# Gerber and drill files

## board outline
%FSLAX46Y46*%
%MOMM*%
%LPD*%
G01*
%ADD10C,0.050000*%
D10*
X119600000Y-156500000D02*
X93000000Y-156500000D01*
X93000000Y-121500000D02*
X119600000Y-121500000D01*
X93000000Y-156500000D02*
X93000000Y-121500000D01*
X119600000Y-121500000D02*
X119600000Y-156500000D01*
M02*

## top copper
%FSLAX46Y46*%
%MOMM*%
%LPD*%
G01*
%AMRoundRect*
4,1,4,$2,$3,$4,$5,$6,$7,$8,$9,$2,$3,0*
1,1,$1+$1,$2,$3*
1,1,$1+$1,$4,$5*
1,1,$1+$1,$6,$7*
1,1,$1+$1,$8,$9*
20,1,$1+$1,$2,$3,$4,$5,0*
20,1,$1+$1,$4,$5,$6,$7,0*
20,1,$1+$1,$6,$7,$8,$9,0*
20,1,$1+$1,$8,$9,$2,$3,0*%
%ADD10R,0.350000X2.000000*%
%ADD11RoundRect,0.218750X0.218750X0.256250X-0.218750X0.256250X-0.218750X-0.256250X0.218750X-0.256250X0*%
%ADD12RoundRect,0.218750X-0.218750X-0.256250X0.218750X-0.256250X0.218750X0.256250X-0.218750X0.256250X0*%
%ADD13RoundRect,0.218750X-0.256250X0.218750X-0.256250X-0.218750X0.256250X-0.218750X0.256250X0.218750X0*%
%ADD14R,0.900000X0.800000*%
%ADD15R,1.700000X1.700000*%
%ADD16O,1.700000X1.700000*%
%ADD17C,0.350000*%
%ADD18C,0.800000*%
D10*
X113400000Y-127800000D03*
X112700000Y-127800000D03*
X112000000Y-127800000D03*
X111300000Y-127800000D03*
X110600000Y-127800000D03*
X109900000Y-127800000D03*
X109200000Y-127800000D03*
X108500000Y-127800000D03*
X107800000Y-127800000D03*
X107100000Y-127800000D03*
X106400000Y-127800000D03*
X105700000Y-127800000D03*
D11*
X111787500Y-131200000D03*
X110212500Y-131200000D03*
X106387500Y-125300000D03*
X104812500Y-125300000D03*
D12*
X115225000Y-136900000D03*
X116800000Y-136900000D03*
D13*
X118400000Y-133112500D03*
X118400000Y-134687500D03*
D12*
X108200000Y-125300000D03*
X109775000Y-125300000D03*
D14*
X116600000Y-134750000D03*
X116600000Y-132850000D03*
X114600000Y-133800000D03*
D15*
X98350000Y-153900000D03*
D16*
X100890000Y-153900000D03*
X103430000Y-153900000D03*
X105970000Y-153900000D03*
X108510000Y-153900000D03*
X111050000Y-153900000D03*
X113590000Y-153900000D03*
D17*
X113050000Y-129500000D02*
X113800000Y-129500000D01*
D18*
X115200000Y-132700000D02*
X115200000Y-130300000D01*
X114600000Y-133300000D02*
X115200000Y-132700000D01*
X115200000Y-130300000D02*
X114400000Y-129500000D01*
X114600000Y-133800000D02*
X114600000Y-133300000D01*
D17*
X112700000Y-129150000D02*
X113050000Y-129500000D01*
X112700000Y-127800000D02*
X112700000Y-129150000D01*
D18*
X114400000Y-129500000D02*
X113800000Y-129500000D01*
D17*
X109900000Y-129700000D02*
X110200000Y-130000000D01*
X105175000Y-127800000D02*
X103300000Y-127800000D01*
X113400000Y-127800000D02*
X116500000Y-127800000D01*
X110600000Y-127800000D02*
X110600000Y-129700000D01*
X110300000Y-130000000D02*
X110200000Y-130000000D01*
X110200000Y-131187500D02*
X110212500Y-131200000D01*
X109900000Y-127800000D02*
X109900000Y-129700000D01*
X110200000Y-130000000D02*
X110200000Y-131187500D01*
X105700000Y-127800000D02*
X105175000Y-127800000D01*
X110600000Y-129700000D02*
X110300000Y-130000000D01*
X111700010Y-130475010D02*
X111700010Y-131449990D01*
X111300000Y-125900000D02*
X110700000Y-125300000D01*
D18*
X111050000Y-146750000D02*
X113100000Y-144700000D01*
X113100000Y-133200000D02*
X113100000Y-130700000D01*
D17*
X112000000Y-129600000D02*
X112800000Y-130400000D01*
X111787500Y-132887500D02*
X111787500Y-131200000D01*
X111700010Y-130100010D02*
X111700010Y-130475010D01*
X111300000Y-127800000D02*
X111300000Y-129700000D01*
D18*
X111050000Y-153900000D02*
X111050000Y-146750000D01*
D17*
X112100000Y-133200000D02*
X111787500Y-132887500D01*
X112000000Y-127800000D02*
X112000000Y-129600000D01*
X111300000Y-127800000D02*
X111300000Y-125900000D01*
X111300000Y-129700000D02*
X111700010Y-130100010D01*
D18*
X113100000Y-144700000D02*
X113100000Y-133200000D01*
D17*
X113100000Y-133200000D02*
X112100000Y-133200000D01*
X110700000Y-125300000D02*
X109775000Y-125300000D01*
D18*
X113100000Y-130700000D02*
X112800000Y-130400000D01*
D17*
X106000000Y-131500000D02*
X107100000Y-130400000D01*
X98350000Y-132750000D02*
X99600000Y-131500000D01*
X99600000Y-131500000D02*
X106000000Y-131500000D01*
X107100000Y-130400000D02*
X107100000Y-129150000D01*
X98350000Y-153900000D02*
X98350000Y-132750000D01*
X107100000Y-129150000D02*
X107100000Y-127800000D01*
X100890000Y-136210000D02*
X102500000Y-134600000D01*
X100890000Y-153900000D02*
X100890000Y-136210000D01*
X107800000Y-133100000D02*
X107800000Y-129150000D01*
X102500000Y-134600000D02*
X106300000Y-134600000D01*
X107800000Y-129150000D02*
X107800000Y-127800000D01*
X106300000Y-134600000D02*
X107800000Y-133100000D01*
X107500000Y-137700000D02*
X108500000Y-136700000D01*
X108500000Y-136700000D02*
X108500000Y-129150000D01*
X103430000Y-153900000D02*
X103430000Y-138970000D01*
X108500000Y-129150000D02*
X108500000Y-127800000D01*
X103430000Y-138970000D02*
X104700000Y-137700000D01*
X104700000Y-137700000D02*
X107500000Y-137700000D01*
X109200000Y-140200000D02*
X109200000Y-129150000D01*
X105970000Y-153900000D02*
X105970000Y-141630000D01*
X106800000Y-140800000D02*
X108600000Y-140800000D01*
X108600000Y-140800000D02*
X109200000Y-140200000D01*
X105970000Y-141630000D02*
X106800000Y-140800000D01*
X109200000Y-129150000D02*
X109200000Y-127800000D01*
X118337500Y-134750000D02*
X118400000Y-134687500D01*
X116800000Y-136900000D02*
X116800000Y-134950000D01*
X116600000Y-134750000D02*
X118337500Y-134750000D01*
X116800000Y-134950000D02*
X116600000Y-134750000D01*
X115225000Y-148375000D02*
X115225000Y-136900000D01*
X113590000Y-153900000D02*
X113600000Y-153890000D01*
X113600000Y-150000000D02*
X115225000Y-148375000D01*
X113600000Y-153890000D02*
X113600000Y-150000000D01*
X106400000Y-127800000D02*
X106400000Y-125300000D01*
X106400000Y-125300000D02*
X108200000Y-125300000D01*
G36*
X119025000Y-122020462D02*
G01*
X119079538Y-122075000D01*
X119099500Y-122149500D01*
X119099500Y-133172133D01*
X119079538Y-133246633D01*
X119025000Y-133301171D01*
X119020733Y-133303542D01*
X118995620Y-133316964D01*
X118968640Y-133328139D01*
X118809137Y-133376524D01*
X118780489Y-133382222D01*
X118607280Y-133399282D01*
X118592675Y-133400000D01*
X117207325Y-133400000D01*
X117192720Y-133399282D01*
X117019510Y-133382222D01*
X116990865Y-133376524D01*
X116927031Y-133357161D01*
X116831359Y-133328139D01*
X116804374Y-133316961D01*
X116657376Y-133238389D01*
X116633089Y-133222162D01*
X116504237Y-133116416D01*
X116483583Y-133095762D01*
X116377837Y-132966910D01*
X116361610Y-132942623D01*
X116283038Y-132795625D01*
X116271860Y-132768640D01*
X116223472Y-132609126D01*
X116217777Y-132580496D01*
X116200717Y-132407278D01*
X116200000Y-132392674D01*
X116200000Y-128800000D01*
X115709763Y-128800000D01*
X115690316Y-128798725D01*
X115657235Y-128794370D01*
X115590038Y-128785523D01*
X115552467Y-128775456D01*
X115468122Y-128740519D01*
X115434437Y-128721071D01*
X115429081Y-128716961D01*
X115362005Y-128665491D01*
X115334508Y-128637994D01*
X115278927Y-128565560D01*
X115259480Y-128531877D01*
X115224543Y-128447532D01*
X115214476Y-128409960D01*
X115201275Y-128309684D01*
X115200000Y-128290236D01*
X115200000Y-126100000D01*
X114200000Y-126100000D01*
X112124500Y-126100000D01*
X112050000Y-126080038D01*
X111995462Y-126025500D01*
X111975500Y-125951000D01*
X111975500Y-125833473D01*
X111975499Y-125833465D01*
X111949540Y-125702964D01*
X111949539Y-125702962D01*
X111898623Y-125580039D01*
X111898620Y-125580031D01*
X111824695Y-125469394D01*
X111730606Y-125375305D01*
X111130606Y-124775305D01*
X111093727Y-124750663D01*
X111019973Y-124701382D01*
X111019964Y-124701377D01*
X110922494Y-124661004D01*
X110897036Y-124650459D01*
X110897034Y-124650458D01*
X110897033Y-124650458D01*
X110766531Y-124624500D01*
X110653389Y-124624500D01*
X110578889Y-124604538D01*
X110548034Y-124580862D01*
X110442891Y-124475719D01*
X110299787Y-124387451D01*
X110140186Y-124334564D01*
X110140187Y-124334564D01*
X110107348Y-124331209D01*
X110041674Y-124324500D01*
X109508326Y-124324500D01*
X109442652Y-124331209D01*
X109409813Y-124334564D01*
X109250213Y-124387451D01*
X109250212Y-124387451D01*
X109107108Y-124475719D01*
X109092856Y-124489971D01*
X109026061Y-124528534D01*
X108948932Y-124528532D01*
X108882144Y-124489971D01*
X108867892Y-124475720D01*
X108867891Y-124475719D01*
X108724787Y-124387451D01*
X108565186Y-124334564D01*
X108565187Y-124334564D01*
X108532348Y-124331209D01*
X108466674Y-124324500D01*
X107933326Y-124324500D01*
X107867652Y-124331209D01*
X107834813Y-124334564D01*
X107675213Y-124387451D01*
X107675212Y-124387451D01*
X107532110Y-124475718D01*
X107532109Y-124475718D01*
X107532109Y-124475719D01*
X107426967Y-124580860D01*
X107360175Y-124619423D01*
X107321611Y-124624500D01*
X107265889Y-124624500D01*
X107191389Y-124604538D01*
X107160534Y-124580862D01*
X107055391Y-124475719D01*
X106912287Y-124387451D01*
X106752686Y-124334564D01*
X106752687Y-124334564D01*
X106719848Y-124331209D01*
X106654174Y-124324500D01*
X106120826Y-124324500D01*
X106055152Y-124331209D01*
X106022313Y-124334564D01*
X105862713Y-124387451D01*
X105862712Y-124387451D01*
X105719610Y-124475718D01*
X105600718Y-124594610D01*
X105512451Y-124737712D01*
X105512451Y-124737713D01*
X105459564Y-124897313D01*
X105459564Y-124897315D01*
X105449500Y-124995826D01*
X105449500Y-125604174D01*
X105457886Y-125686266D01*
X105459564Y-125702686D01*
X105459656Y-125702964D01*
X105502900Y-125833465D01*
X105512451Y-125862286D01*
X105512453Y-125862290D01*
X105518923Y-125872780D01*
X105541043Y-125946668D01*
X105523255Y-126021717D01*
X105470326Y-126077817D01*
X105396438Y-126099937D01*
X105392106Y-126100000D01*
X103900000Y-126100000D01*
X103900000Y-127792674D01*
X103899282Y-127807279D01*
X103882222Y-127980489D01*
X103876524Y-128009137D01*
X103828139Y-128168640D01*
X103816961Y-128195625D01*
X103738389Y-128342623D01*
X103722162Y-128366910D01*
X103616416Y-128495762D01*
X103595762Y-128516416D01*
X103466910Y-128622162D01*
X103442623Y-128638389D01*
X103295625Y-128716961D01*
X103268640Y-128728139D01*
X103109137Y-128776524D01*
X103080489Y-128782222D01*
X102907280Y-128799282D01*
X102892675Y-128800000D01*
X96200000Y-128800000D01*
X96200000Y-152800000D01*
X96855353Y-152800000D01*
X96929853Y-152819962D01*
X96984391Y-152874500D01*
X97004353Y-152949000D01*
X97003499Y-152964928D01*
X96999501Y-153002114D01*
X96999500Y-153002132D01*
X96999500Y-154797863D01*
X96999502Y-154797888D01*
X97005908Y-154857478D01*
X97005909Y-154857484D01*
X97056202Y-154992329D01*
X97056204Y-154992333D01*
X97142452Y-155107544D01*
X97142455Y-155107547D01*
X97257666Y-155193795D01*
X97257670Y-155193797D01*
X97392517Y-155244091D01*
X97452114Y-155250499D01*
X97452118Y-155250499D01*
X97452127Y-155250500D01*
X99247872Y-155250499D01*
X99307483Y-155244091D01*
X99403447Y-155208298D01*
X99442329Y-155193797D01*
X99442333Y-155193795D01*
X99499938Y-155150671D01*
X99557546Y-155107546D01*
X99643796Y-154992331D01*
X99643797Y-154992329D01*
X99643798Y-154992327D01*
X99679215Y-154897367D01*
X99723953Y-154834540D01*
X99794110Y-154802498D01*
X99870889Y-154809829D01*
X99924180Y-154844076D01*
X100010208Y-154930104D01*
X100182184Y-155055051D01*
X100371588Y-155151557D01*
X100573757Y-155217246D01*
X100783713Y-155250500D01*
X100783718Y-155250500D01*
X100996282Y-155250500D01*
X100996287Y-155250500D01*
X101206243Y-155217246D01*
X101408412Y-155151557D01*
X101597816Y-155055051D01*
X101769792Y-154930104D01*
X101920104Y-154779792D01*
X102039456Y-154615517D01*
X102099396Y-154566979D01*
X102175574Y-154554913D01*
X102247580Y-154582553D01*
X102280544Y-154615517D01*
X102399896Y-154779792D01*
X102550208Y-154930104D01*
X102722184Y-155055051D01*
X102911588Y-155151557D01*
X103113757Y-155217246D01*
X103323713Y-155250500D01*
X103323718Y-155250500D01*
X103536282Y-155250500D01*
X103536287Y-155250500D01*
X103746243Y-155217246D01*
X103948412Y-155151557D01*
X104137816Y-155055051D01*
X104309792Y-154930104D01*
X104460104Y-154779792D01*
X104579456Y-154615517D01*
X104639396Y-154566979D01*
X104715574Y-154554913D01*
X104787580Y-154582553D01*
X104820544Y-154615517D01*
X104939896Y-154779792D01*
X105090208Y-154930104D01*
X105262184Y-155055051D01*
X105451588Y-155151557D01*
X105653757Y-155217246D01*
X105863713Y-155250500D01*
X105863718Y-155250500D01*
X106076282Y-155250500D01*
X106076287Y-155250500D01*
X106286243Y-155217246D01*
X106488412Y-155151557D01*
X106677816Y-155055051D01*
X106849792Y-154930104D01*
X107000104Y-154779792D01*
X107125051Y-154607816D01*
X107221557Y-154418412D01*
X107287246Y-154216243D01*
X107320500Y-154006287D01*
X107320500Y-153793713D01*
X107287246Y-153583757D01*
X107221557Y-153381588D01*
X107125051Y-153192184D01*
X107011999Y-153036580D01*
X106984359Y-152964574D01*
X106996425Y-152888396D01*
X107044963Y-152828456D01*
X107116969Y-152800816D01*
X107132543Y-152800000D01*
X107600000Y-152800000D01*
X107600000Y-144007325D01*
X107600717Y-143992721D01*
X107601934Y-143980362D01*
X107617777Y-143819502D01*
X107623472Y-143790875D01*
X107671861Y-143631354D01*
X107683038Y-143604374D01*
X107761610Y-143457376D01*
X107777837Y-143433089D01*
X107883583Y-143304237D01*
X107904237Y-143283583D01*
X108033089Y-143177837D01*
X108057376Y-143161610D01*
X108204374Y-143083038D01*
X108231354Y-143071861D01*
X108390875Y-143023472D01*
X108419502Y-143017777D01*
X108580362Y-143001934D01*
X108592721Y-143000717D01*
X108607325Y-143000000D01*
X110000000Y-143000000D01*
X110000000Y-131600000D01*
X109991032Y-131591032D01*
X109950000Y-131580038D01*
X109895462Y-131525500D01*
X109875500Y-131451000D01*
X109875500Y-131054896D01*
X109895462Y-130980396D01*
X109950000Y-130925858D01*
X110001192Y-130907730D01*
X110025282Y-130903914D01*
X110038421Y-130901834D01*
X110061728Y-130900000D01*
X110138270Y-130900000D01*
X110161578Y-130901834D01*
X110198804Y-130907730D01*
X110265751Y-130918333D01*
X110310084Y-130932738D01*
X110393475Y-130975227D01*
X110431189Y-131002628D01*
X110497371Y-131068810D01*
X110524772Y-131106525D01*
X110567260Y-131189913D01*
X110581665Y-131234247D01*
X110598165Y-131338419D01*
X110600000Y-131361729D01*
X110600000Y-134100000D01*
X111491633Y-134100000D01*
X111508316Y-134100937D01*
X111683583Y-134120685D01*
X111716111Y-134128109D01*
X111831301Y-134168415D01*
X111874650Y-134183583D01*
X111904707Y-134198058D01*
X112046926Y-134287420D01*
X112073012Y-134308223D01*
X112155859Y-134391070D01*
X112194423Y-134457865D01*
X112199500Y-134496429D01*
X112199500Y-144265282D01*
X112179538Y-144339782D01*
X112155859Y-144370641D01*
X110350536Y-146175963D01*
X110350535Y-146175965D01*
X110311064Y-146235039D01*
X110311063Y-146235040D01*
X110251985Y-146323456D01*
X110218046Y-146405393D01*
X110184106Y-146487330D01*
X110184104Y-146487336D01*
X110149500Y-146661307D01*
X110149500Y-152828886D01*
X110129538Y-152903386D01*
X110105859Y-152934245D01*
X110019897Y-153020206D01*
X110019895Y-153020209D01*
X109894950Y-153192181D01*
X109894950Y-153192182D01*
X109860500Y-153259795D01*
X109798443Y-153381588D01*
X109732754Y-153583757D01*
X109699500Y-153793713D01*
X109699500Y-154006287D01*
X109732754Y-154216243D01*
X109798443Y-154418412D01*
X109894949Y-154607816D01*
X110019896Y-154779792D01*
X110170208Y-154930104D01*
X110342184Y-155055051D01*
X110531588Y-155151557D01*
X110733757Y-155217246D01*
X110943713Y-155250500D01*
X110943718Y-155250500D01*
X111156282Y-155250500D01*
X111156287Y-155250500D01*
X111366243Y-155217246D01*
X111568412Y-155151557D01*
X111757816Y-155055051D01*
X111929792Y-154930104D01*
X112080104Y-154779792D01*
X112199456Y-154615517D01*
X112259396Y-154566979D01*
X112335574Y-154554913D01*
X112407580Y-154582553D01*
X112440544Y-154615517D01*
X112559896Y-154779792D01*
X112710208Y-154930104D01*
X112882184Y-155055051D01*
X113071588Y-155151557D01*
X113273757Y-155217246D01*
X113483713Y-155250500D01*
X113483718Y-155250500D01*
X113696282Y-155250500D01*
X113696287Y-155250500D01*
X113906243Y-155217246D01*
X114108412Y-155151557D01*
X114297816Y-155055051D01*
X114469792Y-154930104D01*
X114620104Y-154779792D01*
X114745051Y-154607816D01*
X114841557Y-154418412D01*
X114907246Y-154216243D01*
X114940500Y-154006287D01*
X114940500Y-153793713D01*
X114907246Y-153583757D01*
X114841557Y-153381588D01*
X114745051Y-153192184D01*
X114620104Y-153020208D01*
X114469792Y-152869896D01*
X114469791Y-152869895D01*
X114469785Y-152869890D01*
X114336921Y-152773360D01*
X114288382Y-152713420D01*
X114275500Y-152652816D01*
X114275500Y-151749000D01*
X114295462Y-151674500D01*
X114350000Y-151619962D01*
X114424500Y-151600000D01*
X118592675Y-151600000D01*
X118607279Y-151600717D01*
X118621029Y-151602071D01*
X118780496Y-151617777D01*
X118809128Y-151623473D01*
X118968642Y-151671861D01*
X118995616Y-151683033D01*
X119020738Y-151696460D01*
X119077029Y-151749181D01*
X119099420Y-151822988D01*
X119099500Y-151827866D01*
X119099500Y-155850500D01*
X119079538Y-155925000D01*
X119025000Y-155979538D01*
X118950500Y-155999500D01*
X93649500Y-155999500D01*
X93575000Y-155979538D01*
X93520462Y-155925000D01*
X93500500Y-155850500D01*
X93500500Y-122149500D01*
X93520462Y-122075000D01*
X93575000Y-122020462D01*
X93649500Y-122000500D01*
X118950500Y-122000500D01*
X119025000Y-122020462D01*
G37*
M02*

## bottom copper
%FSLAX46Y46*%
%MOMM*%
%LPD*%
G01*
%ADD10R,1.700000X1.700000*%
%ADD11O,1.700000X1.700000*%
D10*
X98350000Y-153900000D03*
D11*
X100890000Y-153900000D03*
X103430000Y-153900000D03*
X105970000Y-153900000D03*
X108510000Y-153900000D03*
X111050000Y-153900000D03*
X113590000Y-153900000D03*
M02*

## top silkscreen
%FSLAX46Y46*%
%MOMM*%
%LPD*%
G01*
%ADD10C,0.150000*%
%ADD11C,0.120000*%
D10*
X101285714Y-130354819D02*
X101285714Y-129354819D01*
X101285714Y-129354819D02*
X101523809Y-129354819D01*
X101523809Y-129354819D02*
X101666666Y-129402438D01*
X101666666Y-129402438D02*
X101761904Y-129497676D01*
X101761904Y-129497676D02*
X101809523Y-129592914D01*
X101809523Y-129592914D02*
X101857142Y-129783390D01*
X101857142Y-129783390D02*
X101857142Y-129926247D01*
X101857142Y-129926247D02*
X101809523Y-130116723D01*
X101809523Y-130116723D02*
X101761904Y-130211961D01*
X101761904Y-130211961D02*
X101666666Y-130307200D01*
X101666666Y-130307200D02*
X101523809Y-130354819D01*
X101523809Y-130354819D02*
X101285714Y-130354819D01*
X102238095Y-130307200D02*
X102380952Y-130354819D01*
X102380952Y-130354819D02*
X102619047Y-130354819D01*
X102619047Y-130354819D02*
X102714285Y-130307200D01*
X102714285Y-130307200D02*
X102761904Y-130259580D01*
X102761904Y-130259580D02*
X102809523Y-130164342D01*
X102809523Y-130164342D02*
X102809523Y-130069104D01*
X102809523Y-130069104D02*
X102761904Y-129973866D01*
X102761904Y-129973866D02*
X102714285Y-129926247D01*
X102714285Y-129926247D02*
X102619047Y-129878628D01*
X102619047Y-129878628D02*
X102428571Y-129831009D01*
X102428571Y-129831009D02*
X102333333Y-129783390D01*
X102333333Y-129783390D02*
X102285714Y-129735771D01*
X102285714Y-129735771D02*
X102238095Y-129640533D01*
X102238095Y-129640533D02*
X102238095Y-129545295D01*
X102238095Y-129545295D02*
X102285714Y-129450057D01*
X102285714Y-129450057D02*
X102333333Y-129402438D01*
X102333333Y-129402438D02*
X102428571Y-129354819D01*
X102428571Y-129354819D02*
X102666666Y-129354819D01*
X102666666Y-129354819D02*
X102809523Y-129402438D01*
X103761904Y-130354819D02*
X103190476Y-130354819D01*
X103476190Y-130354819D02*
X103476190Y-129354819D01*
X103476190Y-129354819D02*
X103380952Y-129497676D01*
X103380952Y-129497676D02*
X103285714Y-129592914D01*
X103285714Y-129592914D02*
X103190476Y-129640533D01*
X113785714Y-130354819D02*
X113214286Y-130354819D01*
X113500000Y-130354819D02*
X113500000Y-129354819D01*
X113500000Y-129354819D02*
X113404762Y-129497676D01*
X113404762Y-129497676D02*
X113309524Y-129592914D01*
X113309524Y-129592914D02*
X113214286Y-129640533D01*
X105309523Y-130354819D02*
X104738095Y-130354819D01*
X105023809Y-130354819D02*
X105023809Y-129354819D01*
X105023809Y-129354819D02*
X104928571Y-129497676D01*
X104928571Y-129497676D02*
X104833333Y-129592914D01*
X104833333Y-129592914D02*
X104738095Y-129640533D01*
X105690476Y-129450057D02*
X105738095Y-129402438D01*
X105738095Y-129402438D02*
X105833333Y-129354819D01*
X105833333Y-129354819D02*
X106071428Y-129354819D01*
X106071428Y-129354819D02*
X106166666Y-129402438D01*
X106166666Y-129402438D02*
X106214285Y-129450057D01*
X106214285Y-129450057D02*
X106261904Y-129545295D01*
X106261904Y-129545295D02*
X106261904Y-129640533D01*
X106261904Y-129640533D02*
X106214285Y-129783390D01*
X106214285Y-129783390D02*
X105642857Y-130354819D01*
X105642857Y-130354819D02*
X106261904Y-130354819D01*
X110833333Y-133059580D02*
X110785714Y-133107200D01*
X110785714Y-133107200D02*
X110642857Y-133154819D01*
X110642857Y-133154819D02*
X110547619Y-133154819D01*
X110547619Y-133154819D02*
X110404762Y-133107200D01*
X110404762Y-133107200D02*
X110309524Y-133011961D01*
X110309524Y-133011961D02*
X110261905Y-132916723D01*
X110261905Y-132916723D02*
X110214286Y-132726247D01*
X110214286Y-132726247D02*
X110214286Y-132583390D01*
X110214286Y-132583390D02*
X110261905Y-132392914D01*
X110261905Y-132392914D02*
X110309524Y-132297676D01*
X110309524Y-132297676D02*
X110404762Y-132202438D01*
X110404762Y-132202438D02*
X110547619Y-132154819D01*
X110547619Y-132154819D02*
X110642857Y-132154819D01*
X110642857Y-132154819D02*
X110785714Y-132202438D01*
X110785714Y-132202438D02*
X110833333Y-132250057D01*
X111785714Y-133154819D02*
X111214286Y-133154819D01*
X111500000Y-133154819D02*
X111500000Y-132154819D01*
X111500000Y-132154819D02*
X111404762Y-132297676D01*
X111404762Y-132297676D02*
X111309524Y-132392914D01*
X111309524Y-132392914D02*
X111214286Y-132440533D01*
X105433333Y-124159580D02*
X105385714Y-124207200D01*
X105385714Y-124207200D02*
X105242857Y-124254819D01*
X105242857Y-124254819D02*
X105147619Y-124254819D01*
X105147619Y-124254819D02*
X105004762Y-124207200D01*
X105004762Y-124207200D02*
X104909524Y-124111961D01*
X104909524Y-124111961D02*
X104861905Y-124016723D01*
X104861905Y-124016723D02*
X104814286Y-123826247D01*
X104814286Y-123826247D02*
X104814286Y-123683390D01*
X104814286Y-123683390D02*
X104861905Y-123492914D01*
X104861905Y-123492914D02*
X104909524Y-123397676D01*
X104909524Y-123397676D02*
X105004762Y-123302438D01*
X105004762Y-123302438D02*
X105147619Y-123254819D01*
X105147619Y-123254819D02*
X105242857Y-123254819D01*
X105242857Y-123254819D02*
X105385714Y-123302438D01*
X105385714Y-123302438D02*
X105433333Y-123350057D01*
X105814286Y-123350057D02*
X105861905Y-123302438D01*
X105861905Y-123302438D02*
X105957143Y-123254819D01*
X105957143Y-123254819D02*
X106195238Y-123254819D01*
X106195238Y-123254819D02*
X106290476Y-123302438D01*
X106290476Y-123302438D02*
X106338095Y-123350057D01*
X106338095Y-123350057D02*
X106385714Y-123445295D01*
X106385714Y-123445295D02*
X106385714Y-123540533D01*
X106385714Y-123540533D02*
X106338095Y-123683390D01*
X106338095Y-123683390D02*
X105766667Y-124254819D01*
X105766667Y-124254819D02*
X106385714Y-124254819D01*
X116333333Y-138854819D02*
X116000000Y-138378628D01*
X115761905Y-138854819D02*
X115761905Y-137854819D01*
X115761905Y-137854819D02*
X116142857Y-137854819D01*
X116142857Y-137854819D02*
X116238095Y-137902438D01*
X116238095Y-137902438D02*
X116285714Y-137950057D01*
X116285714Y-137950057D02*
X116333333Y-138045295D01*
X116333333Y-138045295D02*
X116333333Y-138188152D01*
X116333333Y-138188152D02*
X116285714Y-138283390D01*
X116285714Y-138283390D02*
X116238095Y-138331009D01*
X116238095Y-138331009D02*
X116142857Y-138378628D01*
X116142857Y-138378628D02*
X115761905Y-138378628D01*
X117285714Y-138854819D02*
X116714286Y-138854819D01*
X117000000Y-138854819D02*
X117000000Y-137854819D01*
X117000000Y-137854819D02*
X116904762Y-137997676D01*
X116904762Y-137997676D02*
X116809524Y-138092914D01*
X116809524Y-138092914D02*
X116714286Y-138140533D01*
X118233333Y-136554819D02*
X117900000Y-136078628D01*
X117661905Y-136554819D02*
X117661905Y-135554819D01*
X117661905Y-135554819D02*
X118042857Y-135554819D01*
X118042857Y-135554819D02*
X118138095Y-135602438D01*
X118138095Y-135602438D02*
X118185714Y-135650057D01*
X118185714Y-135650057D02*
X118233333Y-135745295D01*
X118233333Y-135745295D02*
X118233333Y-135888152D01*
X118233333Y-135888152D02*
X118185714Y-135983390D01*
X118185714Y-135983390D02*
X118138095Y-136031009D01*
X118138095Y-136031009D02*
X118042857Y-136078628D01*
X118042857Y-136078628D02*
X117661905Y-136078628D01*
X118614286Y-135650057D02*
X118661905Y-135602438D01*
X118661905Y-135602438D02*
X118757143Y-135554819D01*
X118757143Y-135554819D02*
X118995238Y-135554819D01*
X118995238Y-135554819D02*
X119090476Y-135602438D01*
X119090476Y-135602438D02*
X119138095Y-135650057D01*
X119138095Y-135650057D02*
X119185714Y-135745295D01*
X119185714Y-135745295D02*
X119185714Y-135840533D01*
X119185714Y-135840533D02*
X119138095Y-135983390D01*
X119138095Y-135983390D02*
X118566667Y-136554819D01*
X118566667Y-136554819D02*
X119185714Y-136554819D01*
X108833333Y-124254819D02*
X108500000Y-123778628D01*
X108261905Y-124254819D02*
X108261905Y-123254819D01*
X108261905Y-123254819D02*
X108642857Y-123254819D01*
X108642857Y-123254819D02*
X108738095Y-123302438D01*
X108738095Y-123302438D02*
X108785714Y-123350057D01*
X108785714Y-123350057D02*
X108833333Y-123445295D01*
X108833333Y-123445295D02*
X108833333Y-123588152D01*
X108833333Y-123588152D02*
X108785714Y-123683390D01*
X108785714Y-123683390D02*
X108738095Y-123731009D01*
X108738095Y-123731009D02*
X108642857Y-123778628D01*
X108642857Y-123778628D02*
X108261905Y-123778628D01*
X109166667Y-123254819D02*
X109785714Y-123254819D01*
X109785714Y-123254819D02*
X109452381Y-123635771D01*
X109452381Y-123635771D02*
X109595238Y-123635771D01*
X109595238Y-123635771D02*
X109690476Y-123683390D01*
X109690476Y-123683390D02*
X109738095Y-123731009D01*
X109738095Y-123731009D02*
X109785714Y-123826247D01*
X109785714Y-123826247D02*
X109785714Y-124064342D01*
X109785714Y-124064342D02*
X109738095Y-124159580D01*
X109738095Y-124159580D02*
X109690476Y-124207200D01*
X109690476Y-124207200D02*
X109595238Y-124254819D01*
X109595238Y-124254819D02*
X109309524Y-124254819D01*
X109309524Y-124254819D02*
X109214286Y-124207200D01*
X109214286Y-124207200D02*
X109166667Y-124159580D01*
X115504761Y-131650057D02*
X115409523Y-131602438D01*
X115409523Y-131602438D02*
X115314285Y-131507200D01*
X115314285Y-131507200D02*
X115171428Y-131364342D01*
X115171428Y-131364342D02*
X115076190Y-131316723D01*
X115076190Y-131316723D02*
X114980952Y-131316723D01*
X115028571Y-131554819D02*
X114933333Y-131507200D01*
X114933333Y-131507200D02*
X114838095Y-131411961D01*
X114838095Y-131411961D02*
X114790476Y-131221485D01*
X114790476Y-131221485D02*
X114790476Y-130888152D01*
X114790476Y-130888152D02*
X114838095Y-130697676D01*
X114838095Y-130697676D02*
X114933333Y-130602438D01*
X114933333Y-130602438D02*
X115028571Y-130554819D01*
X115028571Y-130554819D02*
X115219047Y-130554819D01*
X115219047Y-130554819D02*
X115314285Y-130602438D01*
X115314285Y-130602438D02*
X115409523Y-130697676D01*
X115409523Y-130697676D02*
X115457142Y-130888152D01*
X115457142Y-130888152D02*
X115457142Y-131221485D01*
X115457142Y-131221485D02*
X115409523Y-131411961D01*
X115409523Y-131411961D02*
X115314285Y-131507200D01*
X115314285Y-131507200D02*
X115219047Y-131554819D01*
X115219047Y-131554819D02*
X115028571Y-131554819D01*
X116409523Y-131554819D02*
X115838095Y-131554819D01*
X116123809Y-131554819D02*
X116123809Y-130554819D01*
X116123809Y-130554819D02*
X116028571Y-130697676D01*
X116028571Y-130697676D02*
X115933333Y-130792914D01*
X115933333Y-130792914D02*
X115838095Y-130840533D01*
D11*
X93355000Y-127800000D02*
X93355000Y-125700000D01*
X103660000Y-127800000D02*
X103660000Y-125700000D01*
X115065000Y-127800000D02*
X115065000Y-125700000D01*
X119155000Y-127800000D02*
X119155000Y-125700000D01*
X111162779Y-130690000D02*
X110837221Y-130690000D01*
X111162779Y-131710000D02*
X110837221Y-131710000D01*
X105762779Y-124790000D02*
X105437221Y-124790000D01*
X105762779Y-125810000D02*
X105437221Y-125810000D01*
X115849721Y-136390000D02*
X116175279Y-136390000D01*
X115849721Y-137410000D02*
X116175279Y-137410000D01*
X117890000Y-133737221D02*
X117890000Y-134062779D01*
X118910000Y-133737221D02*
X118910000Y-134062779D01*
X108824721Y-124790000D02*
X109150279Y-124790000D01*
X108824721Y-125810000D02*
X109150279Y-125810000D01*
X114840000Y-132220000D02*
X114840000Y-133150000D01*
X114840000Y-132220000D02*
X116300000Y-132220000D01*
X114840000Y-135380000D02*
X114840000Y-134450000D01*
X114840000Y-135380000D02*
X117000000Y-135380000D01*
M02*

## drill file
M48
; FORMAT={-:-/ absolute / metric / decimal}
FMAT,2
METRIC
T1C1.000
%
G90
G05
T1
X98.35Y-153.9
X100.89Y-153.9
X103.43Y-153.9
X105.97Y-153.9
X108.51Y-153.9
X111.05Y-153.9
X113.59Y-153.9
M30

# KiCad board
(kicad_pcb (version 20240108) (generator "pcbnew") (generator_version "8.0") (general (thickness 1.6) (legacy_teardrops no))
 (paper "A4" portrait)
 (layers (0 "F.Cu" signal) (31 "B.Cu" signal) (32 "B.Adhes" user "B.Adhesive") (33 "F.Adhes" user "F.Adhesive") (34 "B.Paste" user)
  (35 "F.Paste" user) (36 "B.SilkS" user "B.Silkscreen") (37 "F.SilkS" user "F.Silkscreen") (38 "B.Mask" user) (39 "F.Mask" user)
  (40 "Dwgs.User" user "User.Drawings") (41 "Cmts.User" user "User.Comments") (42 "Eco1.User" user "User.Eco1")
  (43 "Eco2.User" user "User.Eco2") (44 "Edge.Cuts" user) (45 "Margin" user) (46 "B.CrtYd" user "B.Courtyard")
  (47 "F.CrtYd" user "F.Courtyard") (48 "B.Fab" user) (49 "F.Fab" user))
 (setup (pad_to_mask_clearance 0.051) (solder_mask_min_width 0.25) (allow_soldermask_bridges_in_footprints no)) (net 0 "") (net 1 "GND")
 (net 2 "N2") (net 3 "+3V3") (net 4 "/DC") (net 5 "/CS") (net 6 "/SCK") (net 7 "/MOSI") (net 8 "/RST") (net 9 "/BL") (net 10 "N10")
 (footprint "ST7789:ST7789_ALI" (layer "F.Cu") (at 109.9 124.3)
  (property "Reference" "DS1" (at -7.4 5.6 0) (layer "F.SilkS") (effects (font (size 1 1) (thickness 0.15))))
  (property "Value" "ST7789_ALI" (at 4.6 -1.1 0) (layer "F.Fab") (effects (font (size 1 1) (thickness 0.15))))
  (fp_line (start -16.545 3.5) (end -16.545 1.4) (stroke (width 0.12) (type solid)) (layer "F.SilkS"))
  (fp_line (start -6.24 3.5) (end -6.24 1.4) (stroke (width 0.12) (type solid)) (layer "F.SilkS"))
  (fp_line (start 5.165 3.5) (end 5.165 1.4) (stroke (width 0.12) (type solid)) (layer "F.SilkS"))
  (fp_line (start 9.255 3.5) (end 9.255 1.4) (stroke (width 0.12) (type solid)) (layer "F.SilkS"))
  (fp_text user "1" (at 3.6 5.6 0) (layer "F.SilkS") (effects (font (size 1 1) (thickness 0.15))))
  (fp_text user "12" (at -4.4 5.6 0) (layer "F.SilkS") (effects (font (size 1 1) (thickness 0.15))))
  (pad "1" smd rect (at 3.5 3.5) (size 0.35 2) (layers "F.Cu" "F.Paste" "F.Mask") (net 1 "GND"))
  (pad "2" smd rect (at 2.8 3.5) (size 0.35 2) (layers "F.Cu" "F.Paste" "F.Mask") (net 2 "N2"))
  (pad "3" smd rect (at 2.1 3.5) (size 0.35 2) (layers "F.Cu" "F.Paste" "F.Mask") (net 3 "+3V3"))
  (pad "4" smd rect (at 1.4 3.5) (size 0.35 2) (layers "F.Cu" "F.Paste" "F.Mask") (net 3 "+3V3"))
  (pad "5" smd rect (at 0.7 3.5) (size 0.35 2) (layers "F.Cu" "F.Paste" "F.Mask") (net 1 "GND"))
  (pad "6" smd rect (at 0 3.5) (size 0.35 2) (layers "F.Cu" "F.Paste" "F.Mask") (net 1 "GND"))
  (pad "7" smd rect (at -0.7 3.5) (size 0.35 2) (layers "F.Cu" "F.Paste" "F.Mask") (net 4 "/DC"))
  (pad "8" smd rect (at -1.4 3.5) (size 0.35 2) (layers "F.Cu" "F.Paste" "F.Mask") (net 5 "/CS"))
  (pad "9" smd rect (at -2.1 3.5) (size 0.35 2) (layers "F.Cu" "F.Paste" "F.Mask") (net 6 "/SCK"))
  (pad "10" smd rect (at -2.8 3.5) (size 0.35 2) (layers "F.Cu" "F.Paste" "F.Mask") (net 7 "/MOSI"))
  (pad "11" smd rect (at -3.5 3.5) (size 0.35 2) (layers "F.Cu" "F.Paste" "F.Mask") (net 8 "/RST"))
  (pad "12" smd rect (at -4.2 3.5) (size 0.35 2) (layers "F.Cu" "F.Paste" "F.Mask") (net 1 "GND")))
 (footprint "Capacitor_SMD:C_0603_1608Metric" (layer "F.Cu") (at 111 131.2 180)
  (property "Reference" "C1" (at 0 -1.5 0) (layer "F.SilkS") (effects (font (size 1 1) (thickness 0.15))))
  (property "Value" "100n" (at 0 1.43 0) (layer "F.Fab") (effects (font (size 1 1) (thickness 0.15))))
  (fp_line (start -0.162779 0.51) (end 0.162779 0.51) (stroke (width 0.12) (type solid)) (layer "F.SilkS"))
  (fp_line (start -0.162779 -0.51) (end 0.162779 -0.51) (stroke (width 0.12) (type solid)) (layer "F.SilkS"))
  (pad "1" smd roundrect (at -0.7875 0 180) (size 0.875 0.95) (layers "F.Cu" "F.Paste" "F.Mask") (roundrect_rratio 0.25) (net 3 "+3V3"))
  (pad "2" smd roundrect (at 0.7875 0 180) (size 0.875 0.95) (layers "F.Cu" "F.Paste" "F.Mask") (roundrect_rratio 0.25) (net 1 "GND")))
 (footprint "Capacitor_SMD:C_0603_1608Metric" (layer "F.Cu") (at 105.6 125.3 180)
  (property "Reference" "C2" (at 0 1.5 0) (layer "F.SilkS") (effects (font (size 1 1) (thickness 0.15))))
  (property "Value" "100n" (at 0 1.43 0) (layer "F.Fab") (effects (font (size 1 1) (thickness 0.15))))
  (fp_line (start -0.162779 0.51) (end 0.162779 0.51) (stroke (width 0.12) (type solid)) (layer "F.SilkS"))
  (fp_line (start -0.162779 -0.51) (end 0.162779 -0.51) (stroke (width 0.12) (type solid)) (layer "F.SilkS"))
  (pad "1" smd roundrect (at -0.7875 0 180) (size 0.875 0.95) (layers "F.Cu" "F.Paste" "F.Mask") (roundrect_rratio 0.25) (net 8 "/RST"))
  (pad "2" smd roundrect (at 0.7875 0 180) (size 0.875 0.95) (layers "F.Cu" "F.Paste" "F.Mask") (roundrect_rratio 0.25) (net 1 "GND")))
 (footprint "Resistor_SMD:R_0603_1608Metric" (layer "F.Cu") (at 116.0125 136.9)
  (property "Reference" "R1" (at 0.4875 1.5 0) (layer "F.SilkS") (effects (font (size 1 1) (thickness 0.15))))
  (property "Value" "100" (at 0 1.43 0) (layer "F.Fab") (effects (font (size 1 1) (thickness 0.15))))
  (fp_line (start -0.162779 -0.51) (end 0.162779 -0.51) (stroke (width 0.12) (type solid)) (layer "F.SilkS"))
  (fp_line (start -0.162779 0.51) (end 0.162779 0.51) (stroke (width 0.12) (type solid)) (layer "F.SilkS"))
  (pad "1" smd roundrect (at -0.7875 0) (size 0.875 0.95) (layers "F.Cu" "F.Paste" "F.Mask") (roundrect_rratio 0.25) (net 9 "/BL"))
  (pad "2" smd roundrect (at 0.7875 0) (size 0.875 0.95) (layers "F.Cu" "F.Paste" "F.Mask") (roundrect_rratio 0.25) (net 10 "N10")))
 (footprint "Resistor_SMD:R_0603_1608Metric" (layer "F.Cu") (at 118.4 133.9 -90)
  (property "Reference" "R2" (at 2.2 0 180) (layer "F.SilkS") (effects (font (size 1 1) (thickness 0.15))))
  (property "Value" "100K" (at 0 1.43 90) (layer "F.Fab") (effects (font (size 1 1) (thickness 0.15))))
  (fp_line (start -0.162779 0.51) (end 0.162779 0.51) (stroke (width 0.12) (type solid)) (layer "F.SilkS"))
  (fp_line (start -0.162779 -0.51) (end 0.162779 -0.51) (stroke (width 0.12) (type solid)) (layer "F.SilkS"))
  (pad "1" smd roundrect (at -0.7875 0 270) (size 0.875 0.95) (layers "F.Cu" "F.Paste" "F.Mask") (roundrect_rratio 0.25) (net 1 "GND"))
  (pad "2" smd roundrect (at 0.7875 0 270) (size 0.875 0.95) (layers "F.Cu" "F.Paste" "F.Mask") (roundrect_rratio 0.25) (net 10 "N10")))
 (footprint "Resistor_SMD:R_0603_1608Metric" (layer "F.Cu") (at 108.9875 125.3)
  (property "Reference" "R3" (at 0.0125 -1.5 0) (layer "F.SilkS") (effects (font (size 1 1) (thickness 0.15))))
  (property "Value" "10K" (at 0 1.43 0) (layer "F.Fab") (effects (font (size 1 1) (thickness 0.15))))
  (fp_line (start -0.162779 -0.51) (end 0.162779 -0.51) (stroke (width 0.12) (type solid)) (layer "F.SilkS"))
  (fp_line (start -0.162779 0.51) (end 0.162779 0.51) (stroke (width 0.12) (type solid)) (layer "F.SilkS"))
  (pad "1" smd roundrect (at -0.7875 0) (size 0.875 0.95) (layers "F.Cu" "F.Paste" "F.Mask") (roundrect_rratio 0.25) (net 8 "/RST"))
  (pad "2" smd roundrect (at 0.7875 0) (size 0.875 0.95) (layers "F.Cu" "F.Paste" "F.Mask") (roundrect_rratio 0.25) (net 3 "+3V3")))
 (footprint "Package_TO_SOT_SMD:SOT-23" (layer "F.Cu") (at 115.6 133.8 180)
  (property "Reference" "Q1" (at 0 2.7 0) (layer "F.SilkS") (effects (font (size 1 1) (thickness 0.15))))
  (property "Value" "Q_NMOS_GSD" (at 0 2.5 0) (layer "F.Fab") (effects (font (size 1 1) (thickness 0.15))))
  (fp_line (start 0.76 1.58) (end 0.76 0.65) (stroke (width 0.12) (type solid)) (layer "F.SilkS"))
  (fp_line (start 0.76 1.58) (end -0.7 1.58) (stroke (width 0.12) (type solid)) (layer "F.SilkS"))
  (fp_line (start 0.76 -1.58) (end 0.76 -0.65) (stroke (width 0.12) (type solid)) (layer "F.SilkS"))
  (fp_line (start 0.76 -1.58) (end -1.4 -1.58) (stroke (width 0.12) (type solid)) (layer "F.SilkS"))
  (pad "1" smd rect (at -1 -0.95 180) (size 0.9 0.8) (layers "F.Cu" "F.Paste" "F.Mask") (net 10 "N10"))
  (pad "2" smd rect (at -1 0.95 180) (size 0.9 0.8) (layers "F.Cu" "F.Paste" "F.Mask") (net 1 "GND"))
  (pad "3" smd rect (at 1 0 180) (size 0.9 0.8) (layers "F.Cu" "F.Paste" "F.Mask") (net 2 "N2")))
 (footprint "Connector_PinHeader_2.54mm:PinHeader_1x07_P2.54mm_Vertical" (layer "B.Cu") (at 98.35 153.9 -90)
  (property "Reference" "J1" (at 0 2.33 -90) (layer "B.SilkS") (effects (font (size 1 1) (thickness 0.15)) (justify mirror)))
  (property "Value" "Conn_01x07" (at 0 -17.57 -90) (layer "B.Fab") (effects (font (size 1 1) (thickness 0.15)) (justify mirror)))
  (pad "1" thru_hole rect (at 0 0 270) (size 1.7 1.7) (drill 1) (layers "*.Cu" "*.Mask") (remove_unused_layers no) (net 7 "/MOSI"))
  (pad "2" thru_hole oval (at 0 -2.54 270) (size 1.7 1.7) (drill 1) (layers "*.Cu" "*.Mask") (remove_unused_layers no) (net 6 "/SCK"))
  (pad "3" thru_hole oval (at 0 -5.08 270) (size 1.7 1.7) (drill 1) (layers "*.Cu" "*.Mask") (remove_unused_layers no) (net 5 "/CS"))
  (pad "4" thru_hole oval (at 0 -7.62 270) (size 1.7 1.7) (drill 1) (layers "*.Cu" "*.Mask") (remove_unused_layers no) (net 4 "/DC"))
  (pad "5" thru_hole oval (at 0 -10.16 270) (size 1.7 1.7) (drill 1) (layers "*.Cu" "*.Mask") (remove_unused_layers no) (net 1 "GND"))
  (pad "6" thru_hole oval (at 0 -12.7 270) (size 1.7 1.7) (drill 1) (layers "*.Cu" "*.Mask") (remove_unused_layers no) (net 3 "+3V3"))
  (pad "7" thru_hole oval (at 0 -15.24 270) (size 1.7 1.7) (drill 1) (layers "*.Cu" "*.Mask") (remove_unused_layers no) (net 9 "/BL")))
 (gr_line (start 119.6 156.5) (end 93 156.5) (stroke (width 0.05) (type solid)) (layer "Edge.Cuts"))
 (gr_line (start 93 121.5) (end 119.6 121.5) (stroke (width 0.05) (type solid)) (layer "Edge.Cuts"))
 (gr_line (start 93 156.5) (end 93 121.5) (stroke (width 0.05) (type solid)) (layer "Edge.Cuts"))
 (gr_line (start 119.6 121.5) (end 119.6 156.5) (stroke (width 0.05) (type solid)) (layer "Edge.Cuts"))
 (segment (start 113.05 129.5) (end 113.8 129.5) (width 0.35) (layer "F.Cu") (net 2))
 (segment (start 115.2 132.7) (end 115.2 130.3) (width 0.8) (layer "F.Cu") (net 2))
 (segment (start 114.6 133.3) (end 115.2 132.7) (width 0.8) (layer "F.Cu") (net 2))
 (segment (start 115.2 130.3) (end 114.4 129.5) (width 0.8) (layer "F.Cu") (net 2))
 (segment (start 114.6 133.8) (end 114.6 133.3) (width 0.8) (layer "F.Cu") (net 2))
 (segment (start 112.7 129.15) (end 113.05 129.5) (width 0.35) (layer "F.Cu") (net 2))
 (segment (start 112.7 127.8) (end 112.7 129.15) (width 0.35) (layer "F.Cu") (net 2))
 (segment (start 114.4 129.5) (end 113.8 129.5) (width 0.8) (layer "F.Cu") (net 2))
 (segment (start 109.9 129.7) (end 110.2 130) (width 0.35) (layer "F.Cu") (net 1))
 (segment (start 105.175 127.8) (end 103.3 127.8) (width 0.35) (layer "F.Cu") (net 1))
 (segment (start 113.4 127.8) (end 116.5 127.8) (width 0.35) (layer "F.Cu") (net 1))
 (segment (start 110.6 127.8) (end 110.6 129.7) (width 0.35) (layer "F.Cu") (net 1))
 (segment (start 110.3 130) (end 110.2 130) (width 0.35) (layer "F.Cu") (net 1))
 (segment (start 110.2 131.1875) (end 110.2125 131.2) (width 0.35) (layer "F.Cu") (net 1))
 (segment (start 109.9 127.8) (end 109.9 129.7) (width 0.35) (layer "F.Cu") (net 1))
 (segment (start 110.2 130) (end 110.2 131.1875) (width 0.35) (layer "F.Cu") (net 1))
 (segment (start 105.7 127.8) (end 105.175 127.8) (width 0.35) (layer "F.Cu") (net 1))
 (segment (start 110.6 129.7) (end 110.3 130) (width 0.35) (layer "F.Cu") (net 1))
 (segment (start 111.70001 130.47501) (end 111.70001 131.44999) (width 0.35) (layer "F.Cu") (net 3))
 (segment (start 111.3 125.9) (end 110.7 125.3) (width 0.35) (layer "F.Cu") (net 3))
 (segment (start 111.05 146.75) (end 113.1 144.7) (width 0.8) (layer "F.Cu") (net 3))
 (segment (start 113.1 133.2) (end 113.1 130.7) (width 0.8) (layer "F.Cu") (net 3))
 (segment (start 112 129.6) (end 112.8 130.4) (width 0.35) (layer "F.Cu") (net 3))
 (segment (start 111.7875 132.8875) (end 111.7875 131.2) (width 0.35) (layer "F.Cu") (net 3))
 (segment (start 111.70001 130.10001) (end 111.70001 130.47501) (width 0.35) (layer "F.Cu") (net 3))
 (segment (start 111.3 127.8) (end 111.3 129.7) (width 0.35) (layer "F.Cu") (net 3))
 (segment (start 111.05 153.9) (end 111.05 146.75) (width 0.8) (layer "F.Cu") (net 3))
 (segment (start 112.1 133.2) (end 111.7875 132.8875) (width 0.35) (layer "F.Cu") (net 3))
 (segment (start 112 127.8) (end 112 129.6) (width 0.35) (layer "F.Cu") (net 3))
 (segment (start 111.3 127.8) (end 111.3 125.9) (width 0.35) (layer "F.Cu") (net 3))
 (segment (start 111.3 129.7) (end 111.70001 130.10001) (width 0.35) (layer "F.Cu") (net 3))
 (segment (start 113.1 144.7) (end 113.1 133.2) (width 0.8) (layer "F.Cu") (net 3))
 (segment (start 113.1 133.2) (end 112.1 133.2) (width 0.35) (layer "F.Cu") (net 3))
 (segment (start 110.7 125.3) (end 109.775 125.3) (width 0.35) (layer "F.Cu") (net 3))
 (segment (start 113.1 130.7) (end 112.8 130.4) (width 0.8) (layer "F.Cu") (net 3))
 (segment (start 106 131.5) (end 107.1 130.4) (width 0.35) (layer "F.Cu") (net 7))
 (segment (start 98.35 132.75) (end 99.6 131.5) (width 0.35) (layer "F.Cu") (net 7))
 (segment (start 99.6 131.5) (end 106 131.5) (width 0.35) (layer "F.Cu") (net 7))
 (segment (start 107.1 130.4) (end 107.1 129.15) (width 0.35) (layer "F.Cu") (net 7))
 (segment (start 98.35 153.9) (end 98.35 132.75) (width 0.35) (layer "F.Cu") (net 7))
 (segment (start 107.1 129.15) (end 107.1 127.8) (width 0.35) (layer "F.Cu") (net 7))
 (segment (start 100.89 136.21) (end 102.5 134.6) (width 0.35) (layer "F.Cu") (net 6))
 (segment (start 100.89 153.9) (end 100.89 136.21) (width 0.35) (layer "F.Cu") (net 6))
 (segment (start 107.8 133.1) (end 107.8 129.15) (width 0.35) (layer "F.Cu") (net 6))
 (segment (start 102.5 134.6) (end 106.3 134.6) (width 0.35) (layer "F.Cu") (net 6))
 (segment (start 107.8 129.15) (end 107.8 127.8) (width 0.35) (layer "F.Cu") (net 6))
 (segment (start 106.3 134.6) (end 107.8 133.1) (width 0.35) (layer "F.Cu") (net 6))
 (segment (start 107.5 137.7) (end 108.5 136.7) (width 0.35) (layer "F.Cu") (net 5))
 (segment (start 108.5 136.7) (end 108.5 129.15) (width 0.35) (layer "F.Cu") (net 5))
 (segment (start 103.43 153.9) (end 103.43 138.97) (width 0.35) (layer "F.Cu") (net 5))
 (segment (start 108.5 129.15) (end 108.5 127.8) (width 0.35) (layer "F.Cu") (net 5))
 (segment (start 103.43 138.97) (end 104.7 137.7) (width 0.35) (layer "F.Cu") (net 5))
 (segment (start 104.7 137.7) (end 107.5 137.7) (width 0.35) (layer "F.Cu") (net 5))
 (segment (start 109.2 140.2) (end 109.2 129.15) (width 0.35) (layer "F.Cu") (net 4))
 (segment (start 105.97 153.9) (end 105.97 141.63) (width 0.35) (layer "F.Cu") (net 4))
 (segment (start 106.8 140.8) (end 108.6 140.8) (width 0.35) (layer "F.Cu") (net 4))
 (segment (start 108.6 140.8) (end 109.2 140.2) (width 0.35) (layer "F.Cu") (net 4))
 (segment (start 105.97 141.63) (end 106.8 140.8) (width 0.35) (layer "F.Cu") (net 4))
 (segment (start 109.2 129.15) (end 109.2 127.8) (width 0.35) (layer "F.Cu") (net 4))
 (segment (start 118.3375 134.75) (end 118.4 134.6875) (width 0.35) (layer "F.Cu") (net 10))
 (segment (start 116.8 136.9) (end 116.8 134.95) (width 0.35) (layer "F.Cu") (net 10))
 (segment (start 116.6 134.75) (end 118.3375 134.75) (width 0.35) (layer "F.Cu") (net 10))
 (segment (start 116.8 134.95) (end 116.6 134.75) (width 0.35) (layer "F.Cu") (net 10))
 (segment (start 115.225 148.375) (end 115.225 136.9) (width 0.35) (layer "F.Cu") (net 9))
 (segment (start 113.59 153.9) (end 113.6 153.89) (width 0.35) (layer "F.Cu") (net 9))
 (segment (start 113.6 150) (end 115.225 148.375) (width 0.35) (layer "F.Cu") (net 9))
 (segment (start 113.6 153.89) (end 113.6 150) (width 0.35) (layer "F.Cu") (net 9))
 (segment (start 106.4 127.8) (end 106.4 125.3) (width 0.35) (layer "F.Cu") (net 8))
 (segment (start 106.4 125.3) (end 108.2 125.3) (width 0.35) (layer "F.Cu") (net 8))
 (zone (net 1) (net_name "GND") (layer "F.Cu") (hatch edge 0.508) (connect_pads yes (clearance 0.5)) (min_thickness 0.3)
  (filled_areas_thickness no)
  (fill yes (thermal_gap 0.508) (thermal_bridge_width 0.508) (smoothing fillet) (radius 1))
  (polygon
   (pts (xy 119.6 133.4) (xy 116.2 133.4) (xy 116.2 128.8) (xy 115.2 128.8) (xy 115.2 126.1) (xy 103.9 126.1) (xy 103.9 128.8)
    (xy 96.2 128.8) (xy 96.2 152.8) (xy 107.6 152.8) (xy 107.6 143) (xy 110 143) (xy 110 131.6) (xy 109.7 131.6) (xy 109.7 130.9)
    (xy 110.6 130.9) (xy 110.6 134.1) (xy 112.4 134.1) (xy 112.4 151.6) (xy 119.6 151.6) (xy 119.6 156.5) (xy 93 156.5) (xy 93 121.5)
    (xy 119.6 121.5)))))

